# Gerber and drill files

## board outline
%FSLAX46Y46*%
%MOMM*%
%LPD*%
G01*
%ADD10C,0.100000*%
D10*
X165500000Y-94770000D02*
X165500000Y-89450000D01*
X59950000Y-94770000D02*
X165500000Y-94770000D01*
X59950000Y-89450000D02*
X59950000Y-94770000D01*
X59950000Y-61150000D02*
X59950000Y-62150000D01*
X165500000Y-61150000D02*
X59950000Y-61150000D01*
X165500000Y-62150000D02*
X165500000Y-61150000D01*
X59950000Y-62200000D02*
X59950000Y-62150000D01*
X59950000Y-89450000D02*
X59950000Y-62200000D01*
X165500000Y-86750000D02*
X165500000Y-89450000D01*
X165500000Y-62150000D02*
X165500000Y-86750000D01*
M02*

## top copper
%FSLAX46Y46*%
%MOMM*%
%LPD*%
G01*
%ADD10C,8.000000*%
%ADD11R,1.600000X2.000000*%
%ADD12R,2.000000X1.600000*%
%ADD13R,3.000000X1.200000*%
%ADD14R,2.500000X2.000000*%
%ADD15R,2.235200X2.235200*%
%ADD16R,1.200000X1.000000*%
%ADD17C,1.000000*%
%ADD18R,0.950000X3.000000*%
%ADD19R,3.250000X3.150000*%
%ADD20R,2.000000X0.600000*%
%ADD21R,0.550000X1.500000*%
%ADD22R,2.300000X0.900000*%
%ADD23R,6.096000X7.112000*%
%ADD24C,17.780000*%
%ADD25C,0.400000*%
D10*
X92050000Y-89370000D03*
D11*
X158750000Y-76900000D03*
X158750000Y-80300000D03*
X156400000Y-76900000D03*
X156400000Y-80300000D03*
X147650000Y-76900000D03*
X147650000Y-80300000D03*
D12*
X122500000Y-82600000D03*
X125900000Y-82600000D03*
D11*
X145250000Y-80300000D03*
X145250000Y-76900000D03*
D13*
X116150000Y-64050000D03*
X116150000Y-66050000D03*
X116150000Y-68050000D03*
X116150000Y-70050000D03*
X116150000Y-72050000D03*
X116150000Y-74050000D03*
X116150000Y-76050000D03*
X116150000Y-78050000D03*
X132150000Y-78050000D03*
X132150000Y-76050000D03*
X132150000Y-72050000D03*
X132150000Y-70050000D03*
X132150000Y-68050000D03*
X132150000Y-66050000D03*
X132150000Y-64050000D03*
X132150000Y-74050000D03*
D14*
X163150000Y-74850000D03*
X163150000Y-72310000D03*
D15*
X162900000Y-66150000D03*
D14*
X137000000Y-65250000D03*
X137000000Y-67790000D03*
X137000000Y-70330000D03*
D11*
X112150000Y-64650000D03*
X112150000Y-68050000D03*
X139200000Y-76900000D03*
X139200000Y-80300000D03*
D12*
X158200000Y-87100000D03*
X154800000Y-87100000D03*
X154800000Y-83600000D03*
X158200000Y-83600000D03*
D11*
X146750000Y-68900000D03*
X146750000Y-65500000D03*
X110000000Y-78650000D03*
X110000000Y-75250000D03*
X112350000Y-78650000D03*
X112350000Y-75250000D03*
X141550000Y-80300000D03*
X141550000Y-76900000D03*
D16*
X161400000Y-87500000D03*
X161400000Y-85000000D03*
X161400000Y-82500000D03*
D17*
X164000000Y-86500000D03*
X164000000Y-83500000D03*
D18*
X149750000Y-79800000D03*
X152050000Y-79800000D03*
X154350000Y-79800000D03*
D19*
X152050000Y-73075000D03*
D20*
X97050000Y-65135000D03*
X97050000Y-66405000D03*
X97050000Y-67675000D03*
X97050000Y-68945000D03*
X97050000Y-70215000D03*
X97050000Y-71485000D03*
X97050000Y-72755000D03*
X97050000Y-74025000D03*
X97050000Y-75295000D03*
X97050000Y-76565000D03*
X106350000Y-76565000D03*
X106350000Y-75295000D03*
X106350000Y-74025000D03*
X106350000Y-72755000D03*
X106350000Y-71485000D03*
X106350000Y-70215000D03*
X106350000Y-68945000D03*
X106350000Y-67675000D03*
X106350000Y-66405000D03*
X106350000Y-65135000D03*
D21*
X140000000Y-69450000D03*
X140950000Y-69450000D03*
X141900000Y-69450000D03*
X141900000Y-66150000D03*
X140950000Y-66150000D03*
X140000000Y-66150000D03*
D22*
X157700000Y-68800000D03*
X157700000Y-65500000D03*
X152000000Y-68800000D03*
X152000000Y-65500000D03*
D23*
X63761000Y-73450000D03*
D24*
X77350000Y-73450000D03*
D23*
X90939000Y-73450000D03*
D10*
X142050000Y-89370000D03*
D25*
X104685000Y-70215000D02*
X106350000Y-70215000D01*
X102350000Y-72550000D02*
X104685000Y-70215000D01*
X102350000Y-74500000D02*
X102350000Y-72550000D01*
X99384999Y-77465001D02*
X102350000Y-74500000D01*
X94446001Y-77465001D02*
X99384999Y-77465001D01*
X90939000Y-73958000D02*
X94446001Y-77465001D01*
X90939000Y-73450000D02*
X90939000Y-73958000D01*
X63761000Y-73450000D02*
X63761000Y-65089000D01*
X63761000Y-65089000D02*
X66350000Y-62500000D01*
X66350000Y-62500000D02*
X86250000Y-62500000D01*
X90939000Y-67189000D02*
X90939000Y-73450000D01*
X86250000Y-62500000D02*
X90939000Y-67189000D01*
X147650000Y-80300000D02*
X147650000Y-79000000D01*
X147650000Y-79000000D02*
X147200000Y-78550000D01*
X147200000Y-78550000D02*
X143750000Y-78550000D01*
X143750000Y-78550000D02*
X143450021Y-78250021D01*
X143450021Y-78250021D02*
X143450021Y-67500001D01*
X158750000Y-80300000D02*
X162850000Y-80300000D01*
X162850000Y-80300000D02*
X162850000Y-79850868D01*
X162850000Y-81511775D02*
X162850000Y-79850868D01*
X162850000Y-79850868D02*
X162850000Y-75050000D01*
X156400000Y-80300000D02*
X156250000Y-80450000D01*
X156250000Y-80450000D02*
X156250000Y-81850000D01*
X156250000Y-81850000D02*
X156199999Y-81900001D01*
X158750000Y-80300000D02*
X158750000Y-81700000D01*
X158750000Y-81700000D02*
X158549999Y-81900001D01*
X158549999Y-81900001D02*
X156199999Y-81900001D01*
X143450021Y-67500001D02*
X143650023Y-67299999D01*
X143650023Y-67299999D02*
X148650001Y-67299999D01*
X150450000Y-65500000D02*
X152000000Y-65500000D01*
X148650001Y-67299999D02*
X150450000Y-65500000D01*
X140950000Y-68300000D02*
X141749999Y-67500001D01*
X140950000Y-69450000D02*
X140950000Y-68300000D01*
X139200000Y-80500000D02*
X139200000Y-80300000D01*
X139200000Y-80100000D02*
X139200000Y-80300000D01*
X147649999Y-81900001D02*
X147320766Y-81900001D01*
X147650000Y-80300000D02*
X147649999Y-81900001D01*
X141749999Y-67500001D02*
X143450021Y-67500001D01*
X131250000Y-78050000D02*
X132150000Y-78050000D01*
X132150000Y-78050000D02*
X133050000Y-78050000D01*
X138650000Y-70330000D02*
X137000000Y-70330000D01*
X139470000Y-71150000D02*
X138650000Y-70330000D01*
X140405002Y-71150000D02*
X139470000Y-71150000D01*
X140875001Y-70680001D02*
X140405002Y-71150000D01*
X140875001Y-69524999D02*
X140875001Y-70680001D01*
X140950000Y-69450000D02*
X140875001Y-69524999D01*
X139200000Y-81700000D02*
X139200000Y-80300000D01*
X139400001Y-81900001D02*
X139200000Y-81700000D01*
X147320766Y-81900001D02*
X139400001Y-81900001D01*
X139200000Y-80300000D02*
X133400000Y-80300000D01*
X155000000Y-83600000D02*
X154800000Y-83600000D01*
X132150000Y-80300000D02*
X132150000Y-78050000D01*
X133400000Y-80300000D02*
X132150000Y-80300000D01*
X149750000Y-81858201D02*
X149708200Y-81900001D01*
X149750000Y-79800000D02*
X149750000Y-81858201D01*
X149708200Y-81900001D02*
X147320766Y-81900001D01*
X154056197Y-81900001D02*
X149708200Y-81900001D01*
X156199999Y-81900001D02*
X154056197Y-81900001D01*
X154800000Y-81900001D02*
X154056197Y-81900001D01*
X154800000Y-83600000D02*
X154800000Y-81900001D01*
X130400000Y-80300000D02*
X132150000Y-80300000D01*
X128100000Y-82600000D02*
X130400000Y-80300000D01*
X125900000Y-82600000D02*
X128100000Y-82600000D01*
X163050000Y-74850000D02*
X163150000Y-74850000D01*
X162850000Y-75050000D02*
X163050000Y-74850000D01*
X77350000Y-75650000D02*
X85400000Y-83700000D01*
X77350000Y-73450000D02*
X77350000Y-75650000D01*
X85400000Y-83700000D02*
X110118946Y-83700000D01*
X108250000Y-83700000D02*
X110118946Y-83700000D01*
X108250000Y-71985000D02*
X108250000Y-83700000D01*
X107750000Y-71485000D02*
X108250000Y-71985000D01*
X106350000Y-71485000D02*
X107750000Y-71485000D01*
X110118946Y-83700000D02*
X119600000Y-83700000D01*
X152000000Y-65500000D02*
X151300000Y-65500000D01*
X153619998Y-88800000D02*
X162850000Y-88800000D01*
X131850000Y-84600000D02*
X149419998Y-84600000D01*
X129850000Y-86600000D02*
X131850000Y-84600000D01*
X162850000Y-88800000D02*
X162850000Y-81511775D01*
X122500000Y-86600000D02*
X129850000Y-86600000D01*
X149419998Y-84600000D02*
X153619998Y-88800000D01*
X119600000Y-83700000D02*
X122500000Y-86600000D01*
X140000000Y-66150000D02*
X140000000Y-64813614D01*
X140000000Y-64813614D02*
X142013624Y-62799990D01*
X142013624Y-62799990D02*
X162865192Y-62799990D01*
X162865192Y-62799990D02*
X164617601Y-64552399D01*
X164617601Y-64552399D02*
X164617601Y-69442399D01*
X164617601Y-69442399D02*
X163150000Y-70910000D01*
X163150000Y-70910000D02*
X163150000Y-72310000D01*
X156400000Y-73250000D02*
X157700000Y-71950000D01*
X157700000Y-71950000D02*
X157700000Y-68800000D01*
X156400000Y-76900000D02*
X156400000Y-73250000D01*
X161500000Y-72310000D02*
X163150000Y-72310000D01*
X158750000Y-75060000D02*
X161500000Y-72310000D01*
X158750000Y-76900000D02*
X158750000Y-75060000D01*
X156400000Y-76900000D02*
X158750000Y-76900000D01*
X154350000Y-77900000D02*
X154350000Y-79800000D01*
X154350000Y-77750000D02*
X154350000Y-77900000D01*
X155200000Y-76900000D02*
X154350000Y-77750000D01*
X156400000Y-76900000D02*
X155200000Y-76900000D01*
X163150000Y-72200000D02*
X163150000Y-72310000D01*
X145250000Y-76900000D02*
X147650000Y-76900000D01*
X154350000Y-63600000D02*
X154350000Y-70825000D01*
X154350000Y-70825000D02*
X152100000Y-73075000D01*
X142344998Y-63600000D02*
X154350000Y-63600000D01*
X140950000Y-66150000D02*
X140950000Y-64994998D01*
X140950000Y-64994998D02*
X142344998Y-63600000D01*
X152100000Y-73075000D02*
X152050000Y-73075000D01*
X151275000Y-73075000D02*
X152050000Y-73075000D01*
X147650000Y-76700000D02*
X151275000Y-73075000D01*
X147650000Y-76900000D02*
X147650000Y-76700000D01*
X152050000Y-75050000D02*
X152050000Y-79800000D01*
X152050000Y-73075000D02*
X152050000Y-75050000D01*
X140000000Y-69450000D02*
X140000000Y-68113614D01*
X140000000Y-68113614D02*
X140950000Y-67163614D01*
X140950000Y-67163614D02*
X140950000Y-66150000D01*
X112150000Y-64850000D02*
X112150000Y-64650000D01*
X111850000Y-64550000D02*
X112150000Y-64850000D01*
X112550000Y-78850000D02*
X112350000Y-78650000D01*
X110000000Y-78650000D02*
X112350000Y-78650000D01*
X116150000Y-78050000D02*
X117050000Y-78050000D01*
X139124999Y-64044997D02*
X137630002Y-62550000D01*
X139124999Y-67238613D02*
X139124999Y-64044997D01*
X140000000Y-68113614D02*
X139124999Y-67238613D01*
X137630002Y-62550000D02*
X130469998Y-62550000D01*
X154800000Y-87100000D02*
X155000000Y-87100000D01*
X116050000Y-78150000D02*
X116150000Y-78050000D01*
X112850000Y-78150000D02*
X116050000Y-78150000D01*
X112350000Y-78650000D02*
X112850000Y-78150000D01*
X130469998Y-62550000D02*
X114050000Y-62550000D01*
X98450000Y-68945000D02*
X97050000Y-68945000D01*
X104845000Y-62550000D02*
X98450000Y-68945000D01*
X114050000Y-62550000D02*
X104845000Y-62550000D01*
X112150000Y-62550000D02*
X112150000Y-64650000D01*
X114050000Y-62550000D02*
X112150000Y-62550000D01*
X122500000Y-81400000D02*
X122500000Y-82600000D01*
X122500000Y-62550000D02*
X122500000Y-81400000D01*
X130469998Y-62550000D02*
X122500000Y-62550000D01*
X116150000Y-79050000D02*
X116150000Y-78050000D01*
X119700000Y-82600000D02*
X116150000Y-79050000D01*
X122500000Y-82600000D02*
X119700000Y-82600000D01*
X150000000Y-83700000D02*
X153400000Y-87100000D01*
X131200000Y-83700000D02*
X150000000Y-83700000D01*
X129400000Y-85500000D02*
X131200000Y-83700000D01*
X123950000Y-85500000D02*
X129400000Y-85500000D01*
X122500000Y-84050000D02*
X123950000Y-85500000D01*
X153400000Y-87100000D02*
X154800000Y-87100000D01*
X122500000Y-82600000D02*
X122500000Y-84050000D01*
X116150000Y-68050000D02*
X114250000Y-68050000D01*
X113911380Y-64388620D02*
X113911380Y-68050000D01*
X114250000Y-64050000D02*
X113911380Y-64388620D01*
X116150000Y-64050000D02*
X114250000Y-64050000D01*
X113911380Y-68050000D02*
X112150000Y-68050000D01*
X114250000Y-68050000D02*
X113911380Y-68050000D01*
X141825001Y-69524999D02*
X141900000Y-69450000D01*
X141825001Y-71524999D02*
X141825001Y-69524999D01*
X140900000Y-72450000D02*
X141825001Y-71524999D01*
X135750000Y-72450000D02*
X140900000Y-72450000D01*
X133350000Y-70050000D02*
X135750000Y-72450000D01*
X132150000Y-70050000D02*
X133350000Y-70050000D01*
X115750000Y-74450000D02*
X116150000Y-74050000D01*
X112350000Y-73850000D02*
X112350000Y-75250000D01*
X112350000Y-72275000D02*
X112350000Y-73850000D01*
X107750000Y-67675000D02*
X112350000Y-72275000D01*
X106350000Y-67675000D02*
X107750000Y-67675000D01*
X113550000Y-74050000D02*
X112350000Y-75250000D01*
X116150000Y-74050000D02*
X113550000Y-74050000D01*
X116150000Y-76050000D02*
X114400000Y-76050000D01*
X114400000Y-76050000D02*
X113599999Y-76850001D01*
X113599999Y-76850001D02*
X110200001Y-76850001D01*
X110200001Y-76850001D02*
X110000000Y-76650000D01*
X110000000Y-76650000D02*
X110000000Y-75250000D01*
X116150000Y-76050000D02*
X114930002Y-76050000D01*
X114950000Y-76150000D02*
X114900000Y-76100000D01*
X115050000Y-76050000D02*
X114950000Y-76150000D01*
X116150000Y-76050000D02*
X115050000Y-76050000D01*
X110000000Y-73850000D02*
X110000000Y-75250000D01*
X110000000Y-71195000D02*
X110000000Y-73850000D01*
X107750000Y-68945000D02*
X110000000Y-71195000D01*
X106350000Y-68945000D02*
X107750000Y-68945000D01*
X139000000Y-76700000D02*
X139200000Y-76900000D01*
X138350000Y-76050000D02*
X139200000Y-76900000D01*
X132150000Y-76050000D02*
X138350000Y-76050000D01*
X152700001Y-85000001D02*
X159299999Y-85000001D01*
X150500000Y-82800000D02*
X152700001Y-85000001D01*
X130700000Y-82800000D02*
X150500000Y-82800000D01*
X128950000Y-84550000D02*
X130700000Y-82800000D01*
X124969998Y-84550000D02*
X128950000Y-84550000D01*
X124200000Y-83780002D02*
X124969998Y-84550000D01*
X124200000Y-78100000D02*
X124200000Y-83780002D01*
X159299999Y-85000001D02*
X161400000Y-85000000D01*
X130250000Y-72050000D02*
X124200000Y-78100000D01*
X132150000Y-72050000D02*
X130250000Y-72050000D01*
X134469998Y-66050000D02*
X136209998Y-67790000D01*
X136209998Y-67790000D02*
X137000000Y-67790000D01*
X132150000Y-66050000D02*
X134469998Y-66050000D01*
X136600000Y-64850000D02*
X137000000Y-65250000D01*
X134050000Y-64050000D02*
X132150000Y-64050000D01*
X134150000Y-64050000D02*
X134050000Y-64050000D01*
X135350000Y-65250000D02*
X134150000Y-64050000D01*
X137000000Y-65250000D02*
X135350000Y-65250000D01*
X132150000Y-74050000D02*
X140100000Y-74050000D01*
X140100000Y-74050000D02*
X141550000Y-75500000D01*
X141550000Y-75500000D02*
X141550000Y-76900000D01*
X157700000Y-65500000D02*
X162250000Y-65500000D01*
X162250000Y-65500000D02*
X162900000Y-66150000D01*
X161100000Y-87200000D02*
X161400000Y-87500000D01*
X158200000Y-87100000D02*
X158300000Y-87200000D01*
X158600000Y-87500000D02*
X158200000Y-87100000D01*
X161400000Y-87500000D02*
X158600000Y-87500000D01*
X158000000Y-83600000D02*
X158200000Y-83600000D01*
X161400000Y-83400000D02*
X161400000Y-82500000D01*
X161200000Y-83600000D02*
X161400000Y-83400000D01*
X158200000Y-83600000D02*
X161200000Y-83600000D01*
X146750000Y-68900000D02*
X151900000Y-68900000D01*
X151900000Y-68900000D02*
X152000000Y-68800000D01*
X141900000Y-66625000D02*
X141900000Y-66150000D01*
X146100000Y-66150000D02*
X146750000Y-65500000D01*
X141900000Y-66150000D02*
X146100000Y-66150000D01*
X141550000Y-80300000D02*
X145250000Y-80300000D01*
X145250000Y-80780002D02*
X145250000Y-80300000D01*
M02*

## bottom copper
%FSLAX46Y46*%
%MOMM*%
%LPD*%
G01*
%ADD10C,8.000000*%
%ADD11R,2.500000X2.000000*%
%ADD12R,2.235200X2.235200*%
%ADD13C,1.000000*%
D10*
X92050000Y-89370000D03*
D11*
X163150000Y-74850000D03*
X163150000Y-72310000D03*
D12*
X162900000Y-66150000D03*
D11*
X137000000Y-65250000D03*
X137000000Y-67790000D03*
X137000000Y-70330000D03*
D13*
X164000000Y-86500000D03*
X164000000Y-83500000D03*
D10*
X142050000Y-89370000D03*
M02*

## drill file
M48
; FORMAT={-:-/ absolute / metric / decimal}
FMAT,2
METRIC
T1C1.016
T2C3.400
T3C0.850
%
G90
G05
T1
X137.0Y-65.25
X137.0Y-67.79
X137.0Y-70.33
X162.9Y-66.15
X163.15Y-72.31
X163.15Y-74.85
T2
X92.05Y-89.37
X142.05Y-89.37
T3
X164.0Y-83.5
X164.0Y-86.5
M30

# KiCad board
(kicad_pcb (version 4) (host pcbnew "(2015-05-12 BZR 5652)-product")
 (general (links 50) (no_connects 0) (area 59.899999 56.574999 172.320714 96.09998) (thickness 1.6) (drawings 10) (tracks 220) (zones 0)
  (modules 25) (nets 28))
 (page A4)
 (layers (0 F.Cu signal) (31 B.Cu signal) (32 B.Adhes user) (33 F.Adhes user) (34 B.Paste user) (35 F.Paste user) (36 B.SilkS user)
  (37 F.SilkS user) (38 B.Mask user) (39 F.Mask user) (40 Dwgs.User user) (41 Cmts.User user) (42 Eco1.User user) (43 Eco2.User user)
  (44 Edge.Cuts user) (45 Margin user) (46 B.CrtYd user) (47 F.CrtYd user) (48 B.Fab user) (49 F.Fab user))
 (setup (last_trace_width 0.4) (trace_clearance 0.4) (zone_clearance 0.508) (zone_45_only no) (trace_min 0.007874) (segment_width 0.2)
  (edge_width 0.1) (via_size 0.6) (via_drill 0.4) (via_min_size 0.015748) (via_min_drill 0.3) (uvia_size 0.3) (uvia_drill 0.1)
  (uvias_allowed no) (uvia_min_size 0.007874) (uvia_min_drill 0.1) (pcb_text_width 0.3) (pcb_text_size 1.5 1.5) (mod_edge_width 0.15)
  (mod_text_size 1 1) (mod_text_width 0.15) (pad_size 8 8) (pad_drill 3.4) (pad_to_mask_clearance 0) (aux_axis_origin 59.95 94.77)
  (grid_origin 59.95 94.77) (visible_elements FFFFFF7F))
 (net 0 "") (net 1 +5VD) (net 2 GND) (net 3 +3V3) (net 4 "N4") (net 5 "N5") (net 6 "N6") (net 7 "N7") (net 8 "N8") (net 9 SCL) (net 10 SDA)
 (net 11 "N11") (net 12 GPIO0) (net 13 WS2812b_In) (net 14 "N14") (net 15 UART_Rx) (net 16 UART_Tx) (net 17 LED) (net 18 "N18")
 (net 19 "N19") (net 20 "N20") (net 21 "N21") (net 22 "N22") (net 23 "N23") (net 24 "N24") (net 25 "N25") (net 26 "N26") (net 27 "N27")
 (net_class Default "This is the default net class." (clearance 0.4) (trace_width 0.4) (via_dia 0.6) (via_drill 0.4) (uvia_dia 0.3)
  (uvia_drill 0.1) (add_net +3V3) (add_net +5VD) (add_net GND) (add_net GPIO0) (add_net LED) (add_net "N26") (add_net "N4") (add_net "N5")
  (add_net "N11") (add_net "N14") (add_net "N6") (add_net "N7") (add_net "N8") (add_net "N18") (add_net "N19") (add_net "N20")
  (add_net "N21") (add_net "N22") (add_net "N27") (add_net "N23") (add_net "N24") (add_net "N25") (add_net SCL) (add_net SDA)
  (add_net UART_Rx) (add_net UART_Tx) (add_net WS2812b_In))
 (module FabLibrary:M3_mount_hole (layer F.Cu) (at 92.05 89.37)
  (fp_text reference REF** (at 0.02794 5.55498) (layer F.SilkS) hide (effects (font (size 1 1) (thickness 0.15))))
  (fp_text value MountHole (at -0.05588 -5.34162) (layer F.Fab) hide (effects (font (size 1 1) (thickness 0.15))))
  (pad 1 thru_hole circle (at 0 0) (size 8 8) (drill 3.4) (layers *.Cu *.Mask F.SilkS)))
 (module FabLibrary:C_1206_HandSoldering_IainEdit (layer F.Cu) (at 158.75 78.6 270)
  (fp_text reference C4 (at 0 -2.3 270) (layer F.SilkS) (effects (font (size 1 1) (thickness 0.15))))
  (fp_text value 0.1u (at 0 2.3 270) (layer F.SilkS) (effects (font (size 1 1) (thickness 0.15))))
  (pad 1 smd rect (at -1.7 0 270) (size 2 1.6) (layers F.Cu F.Paste F.Mask) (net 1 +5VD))
  (pad 2 smd rect (at 1.7 0 270) (size 2 1.6) (layers F.Cu F.Paste F.Mask) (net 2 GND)))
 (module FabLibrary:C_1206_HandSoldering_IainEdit (layer F.Cu) (at 156.4 78.6 270)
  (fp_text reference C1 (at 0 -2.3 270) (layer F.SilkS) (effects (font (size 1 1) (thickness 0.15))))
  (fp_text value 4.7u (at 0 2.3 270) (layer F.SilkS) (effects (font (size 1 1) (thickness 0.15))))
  (pad 1 smd rect (at -1.7 0 270) (size 2 1.6) (layers F.Cu F.Paste F.Mask) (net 1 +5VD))
  (pad 2 smd rect (at 1.7 0 270) (size 2 1.6) (layers F.Cu F.Paste F.Mask) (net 2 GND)))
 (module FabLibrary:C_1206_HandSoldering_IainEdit (layer F.Cu) (at 147.65 78.6 270)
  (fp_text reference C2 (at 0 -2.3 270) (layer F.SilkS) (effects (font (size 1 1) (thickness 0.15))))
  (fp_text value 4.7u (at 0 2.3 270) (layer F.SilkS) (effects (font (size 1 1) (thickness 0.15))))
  (pad 1 smd rect (at -1.7 0 270) (size 2 1.6) (layers F.Cu F.Paste F.Mask) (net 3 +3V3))
  (pad 2 smd rect (at 1.7 0 270) (size 2 1.6) (layers F.Cu F.Paste F.Mask) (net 2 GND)))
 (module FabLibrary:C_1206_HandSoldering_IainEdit (layer F.Cu) (at 124.2 82.6)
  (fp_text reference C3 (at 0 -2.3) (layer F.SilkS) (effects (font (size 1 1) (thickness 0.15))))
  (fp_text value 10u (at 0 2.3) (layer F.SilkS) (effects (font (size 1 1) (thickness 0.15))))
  (pad 1 smd rect (at -1.7 0) (size 2 1.6) (layers F.Cu F.Paste F.Mask) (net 3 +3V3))
  (pad 2 smd rect (at 1.7 0) (size 2 1.6) (layers F.Cu F.Paste F.Mask) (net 2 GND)))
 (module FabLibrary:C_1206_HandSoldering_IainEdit (layer F.Cu) (at 145.25 78.6 90)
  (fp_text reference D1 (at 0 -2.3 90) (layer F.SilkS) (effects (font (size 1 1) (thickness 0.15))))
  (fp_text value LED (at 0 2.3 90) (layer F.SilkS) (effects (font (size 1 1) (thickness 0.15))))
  (pad 1 smd rect (at -1.7 0 90) (size 2 1.6) (layers F.Cu F.Paste F.Mask) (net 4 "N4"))
  (pad 2 smd rect (at 1.7 0 90) (size 2 1.6) (layers F.Cu F.Paste F.Mask) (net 3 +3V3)))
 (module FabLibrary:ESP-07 (layer F.Cu) (at 124.15 70.05 270)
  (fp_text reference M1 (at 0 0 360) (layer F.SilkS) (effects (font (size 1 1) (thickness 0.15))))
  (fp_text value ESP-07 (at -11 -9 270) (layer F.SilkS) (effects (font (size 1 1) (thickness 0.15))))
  (pad 1 smd rect (at -6 8 270) (size 1.2 3) (layers F.Cu F.Paste F.Mask) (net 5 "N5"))
  (pad 2 smd rect (at -4 8 270) (size 1.2 3) (layers F.Cu F.Paste F.Mask) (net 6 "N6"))
  (pad 3 smd rect (at -2 8 270) (size 1.2 3) (layers F.Cu F.Paste F.Mask) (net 5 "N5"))
  (pad 4 smd rect (at 0 8 270) (size 1.2 3) (layers F.Cu F.Paste F.Mask) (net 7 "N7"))
  (pad 5 smd rect (at 2 8 270) (size 1.2 3) (layers F.Cu F.Paste F.Mask) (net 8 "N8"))
  (pad 6 smd rect (at 4 8 270) (size 1.2 3) (layers F.Cu F.Paste F.Mask) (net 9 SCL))
  (pad 7 smd rect (at 6 8 270) (size 1.2 3) (layers F.Cu F.Paste F.Mask) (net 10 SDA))
  (pad 8 smd rect (at 8 8 270) (size 1.2 3) (layers F.Cu F.Paste F.Mask) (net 3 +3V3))
  (pad 9 smd rect (at 8 -8 270) (size 1.2 3) (layers F.Cu F.Paste F.Mask) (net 2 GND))
  (pad 10 smd rect (at 6 -8 270) (size 1.2 3) (layers F.Cu F.Paste F.Mask) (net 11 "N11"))
  (pad 12 smd rect (at 2 -8 270) (size 1.2 3) (layers F.Cu F.Paste F.Mask) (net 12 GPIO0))
  (pad 13 smd rect (at 0 -8 270) (size 1.2 3) (layers F.Cu F.Paste F.Mask) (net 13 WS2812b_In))
  (pad 14 smd rect (at -2 -8 270) (size 1.2 3) (layers F.Cu F.Paste F.Mask) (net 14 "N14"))
  (pad 15 smd rect (at -4 -8 270) (size 1.2 3) (layers F.Cu F.Paste F.Mask) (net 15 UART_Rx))
  (pad 16 smd rect (at -6 -8 270) (size 1.2 3) (layers F.Cu F.Paste F.Mask) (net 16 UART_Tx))
  (pad 11 smd rect (at 4 -8 270) (size 1.2 3) (layers F.Cu F.Paste F.Mask) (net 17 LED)))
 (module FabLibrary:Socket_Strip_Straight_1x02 (layer F.Cu) (at 163.15 74.85 90)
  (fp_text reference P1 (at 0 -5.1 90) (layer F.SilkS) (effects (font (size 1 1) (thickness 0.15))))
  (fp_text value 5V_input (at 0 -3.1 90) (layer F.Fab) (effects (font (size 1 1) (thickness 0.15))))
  (pad 1 thru_hole rect (at 0 0 90) (size 2 2.5) (drill 1.016) (layers *.Mask F.Cu F.SilkS) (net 2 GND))
  (pad 2 thru_hole rect (at 2.54 0 90) (size 2 2.5) (drill 1.016) (layers *.Mask F.Cu F.SilkS) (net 1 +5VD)))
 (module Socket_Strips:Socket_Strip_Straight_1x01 (layer F.Cu) (at 162.9 66.15)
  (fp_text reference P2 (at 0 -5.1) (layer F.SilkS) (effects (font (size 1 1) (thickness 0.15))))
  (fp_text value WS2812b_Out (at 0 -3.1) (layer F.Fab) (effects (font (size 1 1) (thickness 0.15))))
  (pad 1 thru_hole rect (at 0 0) (size 2.2352 2.2352) (drill 1.016) (layers *.Cu *.Mask F.SilkS) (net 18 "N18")))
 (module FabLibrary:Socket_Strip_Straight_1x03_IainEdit (layer F.Cu) (at 137 65.25 270)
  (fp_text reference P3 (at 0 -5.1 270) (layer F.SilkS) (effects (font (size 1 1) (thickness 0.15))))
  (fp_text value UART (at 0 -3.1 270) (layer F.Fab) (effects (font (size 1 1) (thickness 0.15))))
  (pad 1 thru_hole rect (at 0 0 270) (size 2 2.5) (drill 1.016) (layers *.Mask F.Cu F.SilkS) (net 16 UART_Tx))
  (pad 2 thru_hole rect (at 2.54 0 270) (size 2 2.5) (drill 1.016) (layers *.Mask F.Cu F.SilkS) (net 15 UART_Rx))
  (pad 3 thru_hole rect (at 5.08 0 270) (size 2 2.5) (drill 1.016) (layers *.Mask F.Cu F.SilkS) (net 2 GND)))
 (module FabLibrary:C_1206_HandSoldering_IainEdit (layer F.Cu) (at 112.15 66.35 270)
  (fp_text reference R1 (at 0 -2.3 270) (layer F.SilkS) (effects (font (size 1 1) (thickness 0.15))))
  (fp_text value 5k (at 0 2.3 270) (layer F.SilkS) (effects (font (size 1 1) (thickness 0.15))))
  (pad 1 smd rect (at -1.7 0 270) (size 2 1.6) (layers F.Cu F.Paste F.Mask) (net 3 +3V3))
  (pad 2 smd rect (at 1.7 0 270) (size 2 1.6) (layers F.Cu F.Paste F.Mask) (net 5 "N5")))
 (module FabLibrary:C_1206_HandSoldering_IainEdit (layer F.Cu) (at 139.2 78.6 270)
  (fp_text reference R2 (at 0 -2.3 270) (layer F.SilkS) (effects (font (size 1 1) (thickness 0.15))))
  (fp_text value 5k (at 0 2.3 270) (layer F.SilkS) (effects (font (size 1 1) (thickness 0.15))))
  (pad 1 smd rect (at -1.7 0 270) (size 2 1.6) (layers F.Cu F.Paste F.Mask) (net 11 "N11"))
  (pad 2 smd rect (at 1.7 0 270) (size 2 1.6) (layers F.Cu F.Paste F.Mask) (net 2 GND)))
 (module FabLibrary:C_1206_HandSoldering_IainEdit (layer F.Cu) (at 156.5 87.1 180)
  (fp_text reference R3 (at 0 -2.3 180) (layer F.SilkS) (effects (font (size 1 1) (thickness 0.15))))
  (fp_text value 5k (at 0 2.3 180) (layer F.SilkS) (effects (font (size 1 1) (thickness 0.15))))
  (pad 1 smd rect (at -1.7 0 180) (size 2 1.6) (layers F.Cu F.Paste F.Mask) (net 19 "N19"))
  (pad 2 smd rect (at 1.7 0 180) (size 2 1.6) (layers F.Cu F.Paste F.Mask) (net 3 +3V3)))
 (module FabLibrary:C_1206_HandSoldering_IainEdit (layer F.Cu) (at 156.5 83.6)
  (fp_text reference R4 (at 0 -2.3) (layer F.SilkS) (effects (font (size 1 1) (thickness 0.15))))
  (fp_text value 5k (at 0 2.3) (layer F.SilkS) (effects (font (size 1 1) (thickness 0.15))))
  (pad 1 smd rect (at -1.7 0) (size 2 1.6) (layers F.Cu F.Paste F.Mask) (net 2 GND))
  (pad 2 smd rect (at 1.7 0) (size 2 1.6) (layers F.Cu F.Paste F.Mask) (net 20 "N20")))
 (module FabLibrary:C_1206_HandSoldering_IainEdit (layer F.Cu) (at 146.75 67.2 90)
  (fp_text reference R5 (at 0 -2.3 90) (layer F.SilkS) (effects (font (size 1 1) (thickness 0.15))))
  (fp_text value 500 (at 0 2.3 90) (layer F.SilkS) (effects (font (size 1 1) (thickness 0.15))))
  (pad 1 smd rect (at -1.7 0 90) (size 2 1.6) (layers F.Cu F.Paste F.Mask) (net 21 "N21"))
  (pad 2 smd rect (at 1.7 0 90) (size 2 1.6) (layers F.Cu F.Paste F.Mask) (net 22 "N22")))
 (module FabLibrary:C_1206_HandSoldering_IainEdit (layer F.Cu) (at 110 76.95 90)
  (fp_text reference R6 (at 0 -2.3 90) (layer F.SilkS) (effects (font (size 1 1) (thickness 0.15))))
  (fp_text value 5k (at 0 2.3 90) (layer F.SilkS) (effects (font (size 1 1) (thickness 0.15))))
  (pad 1 smd rect (at -1.7 0 90) (size 2 1.6) (layers F.Cu F.Paste F.Mask) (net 3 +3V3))
  (pad 2 smd rect (at 1.7 0 90) (size 2 1.6) (layers F.Cu F.Paste F.Mask) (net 10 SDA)))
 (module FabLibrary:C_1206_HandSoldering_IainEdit (layer F.Cu) (at 112.35 76.95 90)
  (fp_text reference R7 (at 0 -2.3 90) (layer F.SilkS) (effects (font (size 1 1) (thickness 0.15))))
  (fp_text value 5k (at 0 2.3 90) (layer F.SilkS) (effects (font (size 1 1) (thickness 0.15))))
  (pad 1 smd rect (at -1.7 0 90) (size 2 1.6) (layers F.Cu F.Paste F.Mask) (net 3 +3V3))
  (pad 2 smd rect (at 1.7 0 90) (size 2 1.6) (layers F.Cu F.Paste F.Mask) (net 9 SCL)))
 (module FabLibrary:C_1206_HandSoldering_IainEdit (layer F.Cu) (at 141.55 78.6 90)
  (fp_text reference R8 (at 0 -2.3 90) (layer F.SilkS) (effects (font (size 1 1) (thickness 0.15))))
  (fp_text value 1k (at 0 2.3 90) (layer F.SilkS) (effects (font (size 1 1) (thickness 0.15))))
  (pad 1 smd rect (at -1.7 0 90) (size 2 1.6) (layers F.Cu F.Paste F.Mask) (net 4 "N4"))
  (pad 2 smd rect (at 1.7 0 90) (size 2 1.6) (layers F.Cu F.Paste F.Mask) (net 17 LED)))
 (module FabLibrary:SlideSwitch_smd (layer F.Cu) (at 164 85 90)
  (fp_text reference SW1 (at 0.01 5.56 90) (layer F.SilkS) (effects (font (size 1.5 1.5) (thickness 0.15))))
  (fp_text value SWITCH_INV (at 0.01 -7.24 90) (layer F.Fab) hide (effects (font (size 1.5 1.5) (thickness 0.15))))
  (pad 1 smd rect (at -2.5 -2.6 90) (size 1 1.2) (layers F.Cu F.Paste F.Mask) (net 19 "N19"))
  (pad 2 smd rect (at 0 -2.6 90) (size 1 1.2) (layers F.Cu F.Paste F.Mask) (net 12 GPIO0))
  (pad 3 smd rect (at 2.5 -2.6 90) (size 1 1.2) (layers F.Cu F.Paste F.Mask) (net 20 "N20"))
  (pad "" np_thru_hole circle (at -1.5 0 90) (size 1 1) (drill 0.85) (layers *.Cu *.Mask F.SilkS))
  (pad "" np_thru_hole circle (at 1.5 0 90) (size 1 1) (drill 0.85) (layers *.Cu *.Mask F.SilkS)))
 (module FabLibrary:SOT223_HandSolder (layer F.Cu) (at 152.05 78.3)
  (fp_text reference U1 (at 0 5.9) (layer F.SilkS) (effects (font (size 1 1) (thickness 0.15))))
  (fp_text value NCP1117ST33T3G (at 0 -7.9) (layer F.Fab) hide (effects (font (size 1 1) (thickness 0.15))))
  (pad 1 smd rect (at -2.3 1.5) (size 0.95 3) (layers F.Cu F.Paste F.Mask) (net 2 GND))
  (pad 2 smd rect (at 0 1.5) (size 0.95 3) (layers F.Cu F.Paste F.Mask) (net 3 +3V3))
  (pad 3 smd rect (at 2.3 1.5) (size 0.95 3) (layers F.Cu F.Paste F.Mask) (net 1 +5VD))
  (pad 2 smd rect (at 0 -5.225) (size 3.25 3.15) (layers F.Cu F.Paste F.Mask) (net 3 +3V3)))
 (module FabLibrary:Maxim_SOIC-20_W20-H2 (layer F.Cu) (at 101.7 70.85 270)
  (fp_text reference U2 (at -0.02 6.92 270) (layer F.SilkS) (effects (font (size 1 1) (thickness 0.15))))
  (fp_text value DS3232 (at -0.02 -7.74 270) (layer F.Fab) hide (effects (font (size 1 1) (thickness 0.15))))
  (pad 1 smd rect (at -5.715 4.65 270) (size 0.6 2) (layers F.Cu F.Paste F.Mask))
  (pad 2 smd rect (at -4.445 4.65 270) (size 0.6 2) (layers F.Cu F.Paste F.Mask))
  (pad 3 smd rect (at -3.175 4.65 270) (size 0.6 2) (layers F.Cu F.Paste F.Mask) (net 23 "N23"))
  (pad 4 smd rect (at -1.905 4.65 270) (size 0.6 2) (layers F.Cu F.Paste F.Mask) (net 3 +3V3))
  (pad 5 smd rect (at -0.635 4.65 270) (size 0.6 2) (layers F.Cu F.Paste F.Mask) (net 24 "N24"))
  (pad 6 smd rect (at 0.635 4.65 270) (size 0.6 2) (layers F.Cu F.Paste F.Mask) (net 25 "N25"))
  (pad 7 smd rect (at 1.905 4.65 270) (size 0.6 2) (layers F.Cu F.Paste F.Mask))
  (pad 8 smd rect (at 3.175 4.65 270) (size 0.6 2) (layers F.Cu F.Paste F.Mask))
  (pad 9 smd rect (at 4.445 4.65 270) (size 0.6 2) (layers F.Cu F.Paste F.Mask))
  (pad 10 smd rect (at 5.715 4.65 270) (size 0.6 2) (layers F.Cu F.Paste F.Mask))
  (pad 11 smd rect (at 5.715 -4.65 270) (size 0.6 2) (layers F.Cu F.Paste F.Mask))
  (pad 12 smd rect (at 4.445 -4.65 270) (size 0.6 2) (layers F.Cu F.Paste F.Mask))
  (pad 13 smd rect (at 3.175 -4.65 270) (size 0.6 2) (layers F.Cu F.Paste F.Mask))
  (pad 14 smd rect (at 1.905 -4.65 270) (size 0.6 2) (layers F.Cu F.Paste F.Mask))
  (pad 15 smd rect (at 0.635 -4.65 270) (size 0.6 2) (layers F.Cu F.Paste F.Mask) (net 2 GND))
  (pad 16 smd rect (at -0.635 -4.65 270) (size 0.6 2) (layers F.Cu F.Paste F.Mask) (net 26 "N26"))
  (pad 17 smd rect (at -1.905 -4.65 270) (size 0.6 2) (layers F.Cu F.Paste F.Mask) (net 10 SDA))
  (pad 18 smd rect (at -3.175 -4.65 270) (size 0.6 2) (layers F.Cu F.Paste F.Mask) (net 9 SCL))
  (pad 19 smd rect (at -4.445 -4.65 270) (size 0.6 2) (layers F.Cu F.Paste F.Mask))
  (pad 20 smd rect (at -5.715 -4.65 270) (size 0.6 2) (layers F.Cu F.Paste F.Mask) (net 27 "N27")))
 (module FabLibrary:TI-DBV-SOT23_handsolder (layer F.Cu) (at 140.95 67.85)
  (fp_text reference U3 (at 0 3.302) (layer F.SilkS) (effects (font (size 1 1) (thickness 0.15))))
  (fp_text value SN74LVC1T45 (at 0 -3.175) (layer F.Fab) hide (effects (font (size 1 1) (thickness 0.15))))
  (pad 1 smd rect (at -0.95 1.6) (size 0.55 1.5) (layers F.Cu F.Paste F.Mask) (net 3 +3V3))
  (pad 2 smd rect (at 0 1.6) (size 0.55 1.5) (layers F.Cu F.Paste F.Mask) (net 2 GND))
  (pad 3 smd rect (at 0.95 1.6) (size 0.55 1.5) (layers F.Cu F.Paste F.Mask) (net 13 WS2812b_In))
  (pad 4 smd rect (at 0.95 -1.7) (size 0.55 1.5) (layers F.Cu F.Paste F.Mask) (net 22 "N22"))
  (pad 5 smd rect (at 0 -1.7) (size 0.55 1.5) (layers F.Cu F.Paste F.Mask) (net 3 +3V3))
  (pad 6 smd rect (at -0.95 -1.7) (size 0.55 1.5) (layers F.Cu F.Paste F.Mask) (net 1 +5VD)))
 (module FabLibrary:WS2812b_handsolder (layer F.Cu) (at 154.85 67.15 180)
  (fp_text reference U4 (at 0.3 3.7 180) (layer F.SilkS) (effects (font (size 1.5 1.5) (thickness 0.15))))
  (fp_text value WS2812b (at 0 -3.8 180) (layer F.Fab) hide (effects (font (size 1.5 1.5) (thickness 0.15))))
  (pad 1 smd rect (at -2.85 -1.65 180) (size 2.3 0.9) (layers F.Cu F.Paste F.Mask) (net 1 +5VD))
  (pad 2 smd rect (at -2.85 1.65 180) (size 2.3 0.9) (layers F.Cu F.Paste F.Mask) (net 18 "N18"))
  (pad 4 smd rect (at 2.85 -1.65 180) (size 2.3 0.9) (layers F.Cu F.Paste F.Mask) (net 21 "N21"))
  (pad 3 smd rect (at 2.85 1.65 180) (size 2.3 0.9) (layers F.Cu F.Paste F.Mask) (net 2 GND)))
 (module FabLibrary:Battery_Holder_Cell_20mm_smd (layer F.Cu) (at 77.35 73.45 180)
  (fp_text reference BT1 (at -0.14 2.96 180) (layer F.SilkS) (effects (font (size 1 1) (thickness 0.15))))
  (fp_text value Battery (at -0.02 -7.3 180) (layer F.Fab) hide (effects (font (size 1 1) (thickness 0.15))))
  (pad 1 smd rect (at 13.589 0 180) (size 6.096 7.112) (layers F.Cu F.Paste F.Mask) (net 26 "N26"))
  (pad 2 smd circle (at 0 0 180) (size 17.78 17.78) (layers F.Cu F.Paste F.Mask) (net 2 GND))
  (pad 1 smd rect (at -13.589 0 180) (size 6.096 7.112) (layers F.Cu F.Paste F.Mask) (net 26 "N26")))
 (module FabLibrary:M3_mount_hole (layer F.Cu) (at 142.05 89.37)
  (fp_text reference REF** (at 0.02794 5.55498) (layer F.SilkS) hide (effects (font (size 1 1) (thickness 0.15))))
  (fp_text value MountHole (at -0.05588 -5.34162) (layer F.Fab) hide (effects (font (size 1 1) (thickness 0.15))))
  (pad 1 thru_hole circle (at 0 0) (size 8 8) (drill 3.4) (layers *.Cu *.Mask F.SilkS)))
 (gr_line (start 165.5 94.77) (end 165.5 89.45) (angle 90) (layer Edge.Cuts) (width 0.1))
 (gr_line (start 59.95 94.77) (end 165.5 94.77) (angle 90) (layer Edge.Cuts) (width 0.1))
 (gr_line (start 59.95 89.45) (end 59.95 94.77) (angle 90) (layer Edge.Cuts) (width 0.1))
 (gr_line (start 59.95 61.15) (end 59.95 62.15) (angle 90) (layer Edge.Cuts) (width 0.1))
 (gr_line (start 165.5 61.15) (end 59.95 61.15) (angle 90) (layer Edge.Cuts) (width 0.1))
 (gr_line (start 165.5 62.15) (end 165.5 61.15) (angle 90) (layer Edge.Cuts) (width 0.1))
 (gr_line (start 59.95 62.2) (end 59.95 62.15) (layer Edge.Cuts) (width 0.1))
 (gr_line (start 59.95 89.45) (end 59.95 62.2) (layer Edge.Cuts) (width 0.1))
 (gr_line (start 165.5 86.75) (end 165.5 89.45) (layer Edge.Cuts) (width 0.1))
 (gr_line (start 165.5 62.15) (end 165.5 86.75) (layer Edge.Cuts) (width 0.1))
 (segment (start 104.685 70.215) (end 106.35 70.215) (width 0.4) (layer F.Cu) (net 26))
 (segment (start 102.35 72.55) (end 104.685 70.215) (width 0.4) (layer F.Cu) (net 26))
 (segment (start 102.35 74.5) (end 102.35 72.55) (width 0.4) (layer F.Cu) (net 26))
 (segment (start 99.384999 77.465001) (end 102.35 74.5) (width 0.4) (layer F.Cu) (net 26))
 (segment (start 94.446001 77.465001) (end 99.384999 77.465001) (width 0.4) (layer F.Cu) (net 26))
 (segment (start 90.939 73.958) (end 94.446001 77.465001) (width 0.4) (layer F.Cu) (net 26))
 (segment (start 90.939 73.45) (end 90.939 73.958) (width 0.4) (layer F.Cu) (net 26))
 (segment (start 63.761 73.45) (end 63.761 65.089) (width 0.4) (layer F.Cu) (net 26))
 (segment (start 63.761 65.089) (end 66.35 62.5) (width 0.4) (layer F.Cu) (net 26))
 (segment (start 66.35 62.5) (end 86.25 62.5) (width 0.4) (layer F.Cu) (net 26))
 (segment (start 90.939 67.189) (end 90.939 73.45) (width 0.4) (layer F.Cu) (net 26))
 (segment (start 86.25 62.5) (end 90.939 67.189) (width 0.4) (layer F.Cu) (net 26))
 (segment (start 147.65 80.3) (end 147.65 79) (width 0.4) (layer F.Cu) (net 2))
 (segment (start 147.65 79) (end 147.2 78.55) (width 0.4) (layer F.Cu) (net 2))
 (segment (start 147.2 78.55) (end 143.75 78.55) (width 0.4) (layer F.Cu) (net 2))
 (segment (start 143.75 78.55) (end 143.450021 78.250021) (width 0.4) (layer F.Cu) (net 2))
 (segment (start 143.450021 78.250021) (end 143.450021 67.500001) (width 0.4) (layer F.Cu) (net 2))
 (segment (start 158.75 80.3) (end 162.85 80.3) (width 0.4) (layer F.Cu) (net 2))
 (segment (start 162.85 80.3) (end 162.85 79.850868) (width 0.4) (layer F.Cu) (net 2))
 (segment (start 162.85 81.511775) (end 162.85 79.850868) (width 0.4) (layer F.Cu) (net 2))
 (segment (start 162.85 79.850868) (end 162.85 75.05) (width 0.4) (layer F.Cu) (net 2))
 (segment (start 156.4 80.3) (end 156.25 80.45) (width 0.4) (layer F.Cu) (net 2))
 (segment (start 156.25 80.45) (end 156.25 81.85) (width 0.4) (layer F.Cu) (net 2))
 (segment (start 156.25 81.85) (end 156.199999 81.900001) (width 0.4) (layer F.Cu) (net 2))
 (segment (start 158.75 80.3) (end 158.75 81.7) (width 0.4) (layer F.Cu) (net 2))
 (segment (start 158.75 81.7) (end 158.549999 81.900001) (width 0.4) (layer F.Cu) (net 2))
 (segment (start 158.549999 81.900001) (end 156.199999 81.900001) (width 0.4) (layer F.Cu) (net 2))
 (segment (start 143.450021 67.500001) (end 143.650023 67.299999) (width 0.4) (layer F.Cu) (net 2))
 (segment (start 143.650023 67.299999) (end 148.650001 67.299999) (width 0.4) (layer F.Cu) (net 2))
 (segment (start 150.45 65.5) (end 152 65.5) (width 0.4) (layer F.Cu) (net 2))
 (segment (start 148.650001 67.299999) (end 150.45 65.5) (width 0.4) (layer F.Cu) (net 2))
 (segment (start 140.95 68.3) (end 141.749999 67.500001) (width 0.4) (layer F.Cu) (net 2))
 (segment (start 140.95 69.45) (end 140.95 68.3) (width 0.4) (layer F.Cu) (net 2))
 (segment (start 139.2 80.5) (end 139.2 80.3) (width 0.4) (layer F.Cu) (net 2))
 (segment (start 139.2 80.1) (end 139.2 80.3) (width 0.4) (layer F.Cu) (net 2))
 (segment (start 147.649999 81.900001) (end 147.320766 81.900001) (width 0.4) (layer F.Cu) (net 2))
 (segment (start 147.65 80.3) (end 147.649999 81.900001) (width 0.4) (layer F.Cu) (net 2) (status 10))
 (segment (start 141.749999 67.500001) (end 143.450021 67.500001) (width 0.4) (layer F.Cu) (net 2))
 (segment (start 131.25 78.05) (end 132.15 78.05) (width 0.4) (layer F.Cu) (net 2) (status 30))
 (segment (start 132.15 78.05) (end 133.05 78.05) (width 0.4) (layer F.Cu) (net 2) (status 30))
 (segment (start 138.65 70.33) (end 137 70.33) (width 0.4) (layer F.Cu) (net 2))
 (segment (start 139.47 71.15) (end 138.65 70.33) (width 0.4) (layer F.Cu) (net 2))
 (segment (start 140.405002 71.15) (end 139.47 71.15) (width 0.4) (layer F.Cu) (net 2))
 (segment (start 140.875001 70.680001) (end 140.405002 71.15) (width 0.4) (layer F.Cu) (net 2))
 (segment (start 140.875001 69.524999) (end 140.875001 70.680001) (width 0.4) (layer F.Cu) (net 2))
 (segment (start 140.95 69.45) (end 140.875001 69.524999) (width 0.4) (layer F.Cu) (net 2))
 (segment (start 139.2 81.7) (end 139.2 80.3) (width 0.4) (layer F.Cu) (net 2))
 (segment (start 139.400001 81.900001) (end 139.2 81.7) (width 0.4) (layer F.Cu) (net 2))
 (segment (start 147.320766 81.900001) (end 139.400001 81.900001) (width 0.4) (layer F.Cu) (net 2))
 (segment (start 139.2 80.3) (end 133.4 80.3) (width 0.4) (layer F.Cu) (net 2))
 (segment (start 155 83.6) (end 154.8 83.6) (width 0.4) (layer F.Cu) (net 2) (status 30))
 (segment (start 132.15 80.3) (end 132.15 78.05) (width 0.4) (layer F.Cu) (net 2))
 (segment (start 133.4 80.3) (end 132.15 80.3) (width 0.4) (layer F.Cu) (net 2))
 (segment (start 149.75 81.858201) (end 149.7082 81.900001) (width 0.4) (layer F.Cu) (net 2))
 (segment (start 149.75 79.8) (end 149.75 81.858201) (width 0.4) (layer F.Cu) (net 2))
 (segment (start 149.7082 81.900001) (end 147.320766 81.900001) (width 0.4) (layer F.Cu) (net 2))
 (segment (start 154.056197 81.900001) (end 149.7082 81.900001) (width 0.4) (layer F.Cu) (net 2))
 (segment (start 156.199999 81.900001) (end 154.056197 81.900001) (width 0.4) (layer F.Cu) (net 2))
 (segment (start 154.8 81.900001) (end 154.056197 81.900001) (width 0.4) (layer F.Cu) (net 2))
 (segment (start 154.8 83.6) (end 154.8 81.900001) (width 0.4) (layer F.Cu) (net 2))
 (segment (start 130.4 80.3) (end 132.15 80.3) (width 0.4) (layer F.Cu) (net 2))
 (segment (start 128.1 82.6) (end 130.4 80.3) (width 0.4) (layer F.Cu) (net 2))
 (segment (start 125.9 82.6) (end 128.1 82.6) (width 0.4) (layer F.Cu) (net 2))
 (segment (start 163.05 74.85) (end 163.15 74.85) (width 0.4) (layer F.Cu) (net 2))
 (segment (start 162.85 75.05) (end 163.05 74.85) (width 0.4) (layer F.Cu) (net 2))
 (segment (start 77.35 75.65) (end 85.4 83.7) (width 0.4) (layer F.Cu) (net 2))
 (segment (start 77.35 73.45) (end 77.35 75.65) (width 0.4) (layer F.Cu) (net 2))
 (segment (start 85.4 83.7) (end 110.118946 83.7) (width 0.4) (layer F.Cu) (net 2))
 (segment (start 108.25 83.7) (end 110.118946 83.7) (width 0.4) (layer F.Cu) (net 2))
 (segment (start 108.25 71.985) (end 108.25 83.7) (width 0.4) (layer F.Cu) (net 2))
 (segment (start 107.75 71.485) (end 108.25 71.985) (width 0.4) (layer F.Cu) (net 2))
 (segment (start 106.35 71.485) (end 107.75 71.485) (width 0.4) (layer F.Cu) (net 2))
 (segment (start 110.118946 83.7) (end 119.6 83.7) (width 0.4) (layer F.Cu) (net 2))
 (segment (start 152 65.5) (end 151.3 65.5) (width 0.4) (layer F.Cu) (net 2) (status 30))
 (segment (start 153.619998 88.8) (end 162.85 88.8) (width 0.4) (layer F.Cu) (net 2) (status 20))
 (segment (start 131.85 84.6) (end 149.419998 84.6) (width 0.4) (layer F.Cu) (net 2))
 (segment (start 129.85 86.6) (end 131.85 84.6) (width 0.4) (layer F.Cu) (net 2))
 (segment (start 162.85 88.8) (end 162.85 81.511775) (width 0.4) (layer F.Cu) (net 2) (status 10))
 (segment (start 122.5 86.6) (end 129.85 86.6) (width 0.4) (layer F.Cu) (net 2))
 (segment (start 149.419998 84.6) (end 153.619998 88.8) (width 0.4) (layer F.Cu) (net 2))
 (segment (start 119.6 83.7) (end 122.5 86.6) (width 0.4) (layer F.Cu) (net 2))
 (segment (start 140 66.15) (end 140 64.813614) (width 0.4) (layer F.Cu) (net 1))
 (segment (start 140 64.813614) (end 142.013624 62.79999) (width 0.4) (layer F.Cu) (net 1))
 (segment (start 142.013624 62.79999) (end 162.865192 62.79999) (width 0.4) (layer F.Cu) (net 1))
 (segment (start 162.865192 62.79999) (end 164.617601 64.552399) (width 0.4) (layer F.Cu) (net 1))
 (segment (start 164.617601 64.552399) (end 164.617601 69.442399) (width 0.4) (layer F.Cu) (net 1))
 (segment (start 164.617601 69.442399) (end 163.15 70.91) (width 0.4) (layer F.Cu) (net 1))
 (segment (start 163.15 70.91) (end 163.15 72.31) (width 0.4) (layer F.Cu) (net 1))
 (segment (start 156.4 73.25) (end 157.7 71.95) (width 0.4) (layer F.Cu) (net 1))
 (segment (start 157.7 71.95) (end 157.7 68.8) (width 0.4) (layer F.Cu) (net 1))
 (segment (start 156.4 76.9) (end 156.4 73.25) (width 0.4) (layer F.Cu) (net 1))
 (segment (start 161.5 72.31) (end 163.15 72.31) (width 0.4) (layer F.Cu) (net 1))
 (segment (start 158.75 75.06) (end 161.5 72.31) (width 0.4) (layer F.Cu) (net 1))
 (segment (start 158.75 76.9) (end 158.75 75.06) (width 0.4) (layer F.Cu) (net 1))
 (segment (start 156.4 76.9) (end 158.75 76.9) (width 0.4) (layer F.Cu) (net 1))
 (segment (start 154.35 77.9) (end 154.35 79.8) (width 0.4) (layer F.Cu) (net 1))
 (segment (start 154.35 77.75) (end 154.35 77.9) (width 0.4) (layer F.Cu) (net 1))
 (segment (start 155.2 76.9) (end 154.35 77.75) (width 0.4) (layer F.Cu) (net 1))
 (segment (start 156.4 76.9) (end 155.2 76.9) (width 0.4) (layer F.Cu) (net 1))
 (segment (start 163.15 72.2) (end 163.15 72.31) (width 0.4) (layer F.Cu) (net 1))
 (segment (start 145.25 76.9) (end 147.65 76.9) (width 0.4) (layer F.Cu) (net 3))
 (segment (start 154.35 63.6) (end 154.35 70.825) (width 0.4) (layer F.Cu) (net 3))
 (segment (start 154.35 70.825) (end 152.1 73.075) (width 0.4) (layer F.Cu) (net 3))
 (segment (start 142.344998 63.6) (end 154.35 63.6) (width 0.4) (layer F.Cu) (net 3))
 (segment (start 140.95 66.15) (end 140.95 64.994998) (width 0.4) (layer F.Cu) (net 3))
 (segment (start 140.95 64.994998) (end 142.344998 63.6) (width 0.4) (layer F.Cu) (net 3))
 (segment (start 152.1 73.075) (end 152.05 73.075) (width 0.4) (layer F.Cu) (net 3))
 (segment (start 151.275 73.075) (end 152.05 73.075) (width 0.4) (layer F.Cu) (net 3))
 (segment (start 147.65 76.7) (end 151.275 73.075) (width 0.4) (layer F.Cu) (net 3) (status 10))
 (segment (start 147.65 76.9) (end 147.65 76.7) (width 0.4) (layer F.Cu) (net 3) (status 30))
 (segment (start 152.05 75.05) (end 152.05 79.8) (width 0.4) (layer F.Cu) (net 3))
 (segment (start 152.05 73.075) (end 152.05 75.05) (width 0.4) (layer F.Cu) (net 3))
 (segment (start 140 69.45) (end 140 68.113614) (width 0.4) (layer F.Cu) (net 3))
 (segment (start 140 68.113614) (end 140.95 67.163614) (width 0.4) (layer F.Cu) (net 3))
 (segment (start 140.95 67.163614) (end 140.95 66.15) (width 0.4) (layer F.Cu) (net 3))
 (segment (start 112.15 64.85) (end 112.15 64.65) (width 0.4) (layer F.Cu) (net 3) (status 30))
 (segment (start 111.85 64.55) (end 112.15 64.85) (width 0.4) (layer F.Cu) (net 3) (status 30))
 (segment (start 112.55 78.85) (end 112.35 78.65) (width 0.4) (layer F.Cu) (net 3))
 (segment (start 110 78.65) (end 112.35 78.65) (width 0.4) (layer F.Cu) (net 3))
 (segment (start 116.15 78.05) (end 117.05 78.05) (width 0.4) (layer F.Cu) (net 3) (status 30))
 (segment (start 139.124999 64.044997) (end 137.630002 62.55) (width 0.4) (layer F.Cu) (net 3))
 (segment (start 139.124999 67.238613) (end 139.124999 64.044997) (width 0.4) (layer F.Cu) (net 3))
 (segment (start 140 68.113614) (end 139.124999 67.238613) (width 0.4) (layer F.Cu) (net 3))
 (segment (start 137.630002 62.55) (end 130.469998 62.55) (width 0.4) (layer F.Cu) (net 3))
 (segment (start 154.8 87.1) (end 155 87.1) (width 0.4) (layer F.Cu) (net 3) (status 30))
 (segment (start 116.05 78.15) (end 116.15 78.05) (width 0.4) (layer F.Cu) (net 3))
 (segment (start 112.85 78.15) (end 116.05 78.15) (width 0.4) (layer F.Cu) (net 3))
 (segment (start 112.35 78.65) (end 112.85 78.15) (width 0.4) (layer F.Cu) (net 3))
 (segment (start 130.469998 62.55) (end 114.05 62.55) (width 0.4) (layer F.Cu) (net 3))
 (segment (start 98.45 68.945) (end 97.05 68.945) (width 0.4) (layer F.Cu) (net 3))
 (segment (start 104.845 62.55) (end 98.45 68.945) (width 0.4) (layer F.Cu) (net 3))
 (segment (start 114.05 62.55) (end 104.845 62.55) (width 0.4) (layer F.Cu) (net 3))
 (segment (start 112.15 62.55) (end 112.15 64.65) (width 0.4) (layer F.Cu) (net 3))
 (segment (start 114.05 62.55) (end 112.15 62.55) (width 0.4) (layer F.Cu) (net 3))
 (segment (start 122.5 81.4) (end 122.5 82.6) (width 0.4) (layer F.Cu) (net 3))
 (segment (start 122.5 62.55) (end 122.5 81.4) (width 0.4) (layer F.Cu) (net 3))
 (segment (start 130.469998 62.55) (end 122.5 62.55) (width 0.4) (layer F.Cu) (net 3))
 (segment (start 116.15 79.05) (end 116.15 78.05) (width 0.4) (layer F.Cu) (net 3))
 (segment (start 119.7 82.6) (end 116.15 79.05) (width 0.4) (layer F.Cu) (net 3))
 (segment (start 122.5 82.6) (end 119.7 82.6) (width 0.4) (layer F.Cu) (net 3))
 (segment (start 150 83.7) (end 153.4 87.1) (width 0.4) (layer F.Cu) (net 3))
 (segment (start 131.2 83.7) (end 150 83.7) (width 0.4) (layer F.Cu) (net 3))
 (segment (start 129.4 85.5) (end 131.2 83.7) (width 0.4) (layer F.Cu) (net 3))
 (segment (start 123.95 85.5) (end 129.4 85.5) (width 0.4) (layer F.Cu) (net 3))
 (segment (start 122.5 84.05) (end 123.95 85.5) (width 0.4) (layer F.Cu) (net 3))
 (segment (start 153.4 87.1) (end 154.8 87.1) (width 0.4) (layer F.Cu) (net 3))
 (segment (start 122.5 82.6) (end 122.5 84.05) (width 0.4) (layer F.Cu) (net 3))
 (segment (start 116.15 68.05) (end 114.25 68.05) (width 0.4) (layer F.Cu) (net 5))
 (segment (start 113.91138 64.38862) (end 113.91138 68.05) (width 0.4) (layer F.Cu) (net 5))
 (segment (start 114.25 64.05) (end 113.91138 64.38862) (width 0.4) (layer F.Cu) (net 5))
 (segment (start 116.15 64.05) (end 114.25 64.05) (width 0.4) (layer F.Cu) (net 5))
 (segment (start 113.91138 68.05) (end 112.15 68.05) (width 0.4) (layer F.Cu) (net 5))
 (segment (start 114.25 68.05) (end 113.91138 68.05) (width 0.4) (layer F.Cu) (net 5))
 (segment (start 141.825001 69.524999) (end 141.9 69.45) (width 0.4) (layer F.Cu) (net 13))
 (segment (start 141.825001 71.524999) (end 141.825001 69.524999) (width 0.4) (layer F.Cu) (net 13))
 (segment (start 140.9 72.45) (end 141.825001 71.524999) (width 0.4) (layer F.Cu) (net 13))
 (segment (start 135.75 72.45) (end 140.9 72.45) (width 0.4) (layer F.Cu) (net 13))
 (segment (start 133.35 70.05) (end 135.75 72.45) (width 0.4) (layer F.Cu) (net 13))
 (segment (start 132.15 70.05) (end 133.35 70.05) (width 0.4) (layer F.Cu) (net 13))
 (segment (start 115.75 74.45) (end 116.15 74.05) (width 0.4) (layer F.Cu) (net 9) (status 30))
 (segment (start 112.35 73.85) (end 112.35 75.25) (width 0.4) (layer F.Cu) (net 9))
 (segment (start 112.35 72.275) (end 112.35 73.85) (width 0.4) (layer F.Cu) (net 9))
 (segment (start 107.75 67.675) (end 112.35 72.275) (width 0.4) (layer F.Cu) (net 9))
 (segment (start 106.35 67.675) (end 107.75 67.675) (width 0.4) (layer F.Cu) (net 9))
 (segment (start 113.55 74.05) (end 112.35 75.25) (width 0.4) (layer F.Cu) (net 9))
 (segment (start 116.15 74.05) (end 113.55 74.05) (width 0.4) (layer F.Cu) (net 9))
 (segment (start 116.15 76.05) (end 114.4 76.05) (width 0.4) (layer F.Cu) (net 10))
 (segment (start 114.4 76.05) (end 113.599999 76.850001) (width 0.4) (layer F.Cu) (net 10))
 (segment (start 113.599999 76.850001) (end 110.200001 76.850001) (width 0.4) (layer F.Cu) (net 10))
 (segment (start 110.200001 76.850001) (end 110 76.65) (width 0.4) (layer F.Cu) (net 10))
 (segment (start 110 76.65) (end 110 75.25) (width 0.4) (layer F.Cu) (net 10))
 (segment (start 116.15 76.05) (end 114.930002 76.05) (width 0.4) (layer F.Cu) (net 10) (status 30))
 (segment (start 114.95 76.15) (end 114.9 76.1) (width 0.4) (layer F.Cu) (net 10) (status 30))
 (segment (start 115.05 76.05) (end 114.95 76.15) (width 0.4) (layer F.Cu) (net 10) (status 30))
 (segment (start 116.15 76.05) (end 115.05 76.05) (width 0.4) (layer F.Cu) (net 10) (status 30))
 (segment (start 110 73.85) (end 110 75.25) (width 0.4) (layer F.Cu) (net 10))
 (segment (start 110 71.195) (end 110 73.85) (width 0.4) (layer F.Cu) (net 10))
 (segment (start 107.75 68.945) (end 110 71.195) (width 0.4) (layer F.Cu) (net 10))
 (segment (start 106.35 68.945) (end 107.75 68.945) (width 0.4) (layer F.Cu) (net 10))
 (segment (start 139 76.7) (end 139.2 76.9) (width 0.4) (layer F.Cu) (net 11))
 (segment (start 138.35 76.05) (end 139.2 76.9) (width 0.4) (layer F.Cu) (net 11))
 (segment (start 132.15 76.05) (end 138.35 76.05) (width 0.4) (layer F.Cu) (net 11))
 (segment (start 152.700001 85.000001) (end 159.299999 85.000001) (width 0.4) (layer F.Cu) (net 12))
 (segment (start 150.5 82.8) (end 152.700001 85.000001) (width 0.4) (layer F.Cu) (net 12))
 (segment (start 130.7 82.8) (end 150.5 82.8) (width 0.4) (layer F.Cu) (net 12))
 (segment (start 128.95 84.55) (end 130.7 82.8) (width 0.4) (layer F.Cu) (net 12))
 (segment (start 124.969998 84.55) (end 128.95 84.55) (width 0.4) (layer F.Cu) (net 12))
 (segment (start 124.2 83.780002) (end 124.969998 84.55) (width 0.4) (layer F.Cu) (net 12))
 (segment (start 124.2 78.1) (end 124.2 83.780002) (width 0.4) (layer F.Cu) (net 12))
 (segment (start 159.299999 85.000001) (end 161.4 85) (width 0.4) (layer F.Cu) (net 12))
 (segment (start 130.25 72.05) (end 124.2 78.1) (width 0.4) (layer F.Cu) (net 12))
 (segment (start 132.15 72.05) (end 130.25 72.05) (width 0.4) (layer F.Cu) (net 12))
 (segment (start 134.469998 66.05) (end 136.209998 67.79) (width 0.4) (layer F.Cu) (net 15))
 (segment (start 136.209998 67.79) (end 137 67.79) (width 0.4) (layer F.Cu) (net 15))
 (segment (start 132.15 66.05) (end 134.469998 66.05) (width 0.4) (layer F.Cu) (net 15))
 (segment (start 136.6 64.85) (end 137 65.25) (width 0.4) (layer F.Cu) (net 16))
 (segment (start 134.05 64.05) (end 132.15 64.05) (width 0.4) (layer F.Cu) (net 16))
 (segment (start 134.15 64.05) (end 134.05 64.05) (width 0.4) (layer F.Cu) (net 16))
 (segment (start 135.35 65.25) (end 134.15 64.05) (width 0.4) (layer F.Cu) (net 16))
 (segment (start 137 65.25) (end 135.35 65.25) (width 0.4) (layer F.Cu) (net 16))
 (segment (start 132.15 74.05) (end 140.1 74.05) (width 0.4) (layer F.Cu) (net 17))
 (segment (start 140.1 74.05) (end 141.55 75.5) (width 0.4) (layer F.Cu) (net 17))
 (segment (start 141.55 75.5) (end 141.55 76.9) (width 0.4) (layer F.Cu) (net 17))
 (segment (start 157.7 65.5) (end 162.25 65.5) (width 0.4) (layer F.Cu) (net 18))
 (segment (start 162.25 65.5) (end 162.9 66.15) (width 0.4) (layer F.Cu) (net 18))
 (segment (start 161.1 87.2) (end 161.4 87.5) (width 0.4) (layer F.Cu) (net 19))
 (segment (start 158.2 87.1) (end 158.3 87.2) (width 0.4) (layer F.Cu) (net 19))
 (segment (start 158.6 87.5) (end 158.2 87.1) (width 0.4) (layer F.Cu) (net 19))
 (segment (start 161.4 87.5) (end 158.6 87.5) (width 0.4) (layer F.Cu) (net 19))
 (segment (start 158 83.6) (end 158.2 83.6) (width 0.4) (layer F.Cu) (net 20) (status 30))
 (segment (start 161.4 83.4) (end 161.4 82.5) (width 0.4) (layer F.Cu) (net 20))
 (segment (start 161.2 83.6) (end 161.4 83.4) (width 0.4) (layer F.Cu) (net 20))
 (segment (start 158.2 83.6) (end 161.2 83.6) (width 0.4) (layer F.Cu) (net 20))
 (segment (start 146.75 68.9) (end 151.9 68.9) (width 0.4) (layer F.Cu) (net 21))
 (segment (start 151.9 68.9) (end 152 68.8) (width 0.4) (layer F.Cu) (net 21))
 (segment (start 141.9 66.625) (end 141.9 66.15) (width 0.4) (layer F.Cu) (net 22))
 (segment (start 146.1 66.15) (end 146.75 65.5) (width 0.4) (layer F.Cu) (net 22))
 (segment (start 141.9 66.15) (end 146.1 66.15) (width 0.4) (layer F.Cu) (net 22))
 (segment (start 141.55 80.3) (end 145.25 80.3) (width 0.4) (layer F.Cu) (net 4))
 (segment (start 145.25 80.780002) (end 145.25 80.3) (width 0.4) (layer F.Cu) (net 4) (status 30)))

